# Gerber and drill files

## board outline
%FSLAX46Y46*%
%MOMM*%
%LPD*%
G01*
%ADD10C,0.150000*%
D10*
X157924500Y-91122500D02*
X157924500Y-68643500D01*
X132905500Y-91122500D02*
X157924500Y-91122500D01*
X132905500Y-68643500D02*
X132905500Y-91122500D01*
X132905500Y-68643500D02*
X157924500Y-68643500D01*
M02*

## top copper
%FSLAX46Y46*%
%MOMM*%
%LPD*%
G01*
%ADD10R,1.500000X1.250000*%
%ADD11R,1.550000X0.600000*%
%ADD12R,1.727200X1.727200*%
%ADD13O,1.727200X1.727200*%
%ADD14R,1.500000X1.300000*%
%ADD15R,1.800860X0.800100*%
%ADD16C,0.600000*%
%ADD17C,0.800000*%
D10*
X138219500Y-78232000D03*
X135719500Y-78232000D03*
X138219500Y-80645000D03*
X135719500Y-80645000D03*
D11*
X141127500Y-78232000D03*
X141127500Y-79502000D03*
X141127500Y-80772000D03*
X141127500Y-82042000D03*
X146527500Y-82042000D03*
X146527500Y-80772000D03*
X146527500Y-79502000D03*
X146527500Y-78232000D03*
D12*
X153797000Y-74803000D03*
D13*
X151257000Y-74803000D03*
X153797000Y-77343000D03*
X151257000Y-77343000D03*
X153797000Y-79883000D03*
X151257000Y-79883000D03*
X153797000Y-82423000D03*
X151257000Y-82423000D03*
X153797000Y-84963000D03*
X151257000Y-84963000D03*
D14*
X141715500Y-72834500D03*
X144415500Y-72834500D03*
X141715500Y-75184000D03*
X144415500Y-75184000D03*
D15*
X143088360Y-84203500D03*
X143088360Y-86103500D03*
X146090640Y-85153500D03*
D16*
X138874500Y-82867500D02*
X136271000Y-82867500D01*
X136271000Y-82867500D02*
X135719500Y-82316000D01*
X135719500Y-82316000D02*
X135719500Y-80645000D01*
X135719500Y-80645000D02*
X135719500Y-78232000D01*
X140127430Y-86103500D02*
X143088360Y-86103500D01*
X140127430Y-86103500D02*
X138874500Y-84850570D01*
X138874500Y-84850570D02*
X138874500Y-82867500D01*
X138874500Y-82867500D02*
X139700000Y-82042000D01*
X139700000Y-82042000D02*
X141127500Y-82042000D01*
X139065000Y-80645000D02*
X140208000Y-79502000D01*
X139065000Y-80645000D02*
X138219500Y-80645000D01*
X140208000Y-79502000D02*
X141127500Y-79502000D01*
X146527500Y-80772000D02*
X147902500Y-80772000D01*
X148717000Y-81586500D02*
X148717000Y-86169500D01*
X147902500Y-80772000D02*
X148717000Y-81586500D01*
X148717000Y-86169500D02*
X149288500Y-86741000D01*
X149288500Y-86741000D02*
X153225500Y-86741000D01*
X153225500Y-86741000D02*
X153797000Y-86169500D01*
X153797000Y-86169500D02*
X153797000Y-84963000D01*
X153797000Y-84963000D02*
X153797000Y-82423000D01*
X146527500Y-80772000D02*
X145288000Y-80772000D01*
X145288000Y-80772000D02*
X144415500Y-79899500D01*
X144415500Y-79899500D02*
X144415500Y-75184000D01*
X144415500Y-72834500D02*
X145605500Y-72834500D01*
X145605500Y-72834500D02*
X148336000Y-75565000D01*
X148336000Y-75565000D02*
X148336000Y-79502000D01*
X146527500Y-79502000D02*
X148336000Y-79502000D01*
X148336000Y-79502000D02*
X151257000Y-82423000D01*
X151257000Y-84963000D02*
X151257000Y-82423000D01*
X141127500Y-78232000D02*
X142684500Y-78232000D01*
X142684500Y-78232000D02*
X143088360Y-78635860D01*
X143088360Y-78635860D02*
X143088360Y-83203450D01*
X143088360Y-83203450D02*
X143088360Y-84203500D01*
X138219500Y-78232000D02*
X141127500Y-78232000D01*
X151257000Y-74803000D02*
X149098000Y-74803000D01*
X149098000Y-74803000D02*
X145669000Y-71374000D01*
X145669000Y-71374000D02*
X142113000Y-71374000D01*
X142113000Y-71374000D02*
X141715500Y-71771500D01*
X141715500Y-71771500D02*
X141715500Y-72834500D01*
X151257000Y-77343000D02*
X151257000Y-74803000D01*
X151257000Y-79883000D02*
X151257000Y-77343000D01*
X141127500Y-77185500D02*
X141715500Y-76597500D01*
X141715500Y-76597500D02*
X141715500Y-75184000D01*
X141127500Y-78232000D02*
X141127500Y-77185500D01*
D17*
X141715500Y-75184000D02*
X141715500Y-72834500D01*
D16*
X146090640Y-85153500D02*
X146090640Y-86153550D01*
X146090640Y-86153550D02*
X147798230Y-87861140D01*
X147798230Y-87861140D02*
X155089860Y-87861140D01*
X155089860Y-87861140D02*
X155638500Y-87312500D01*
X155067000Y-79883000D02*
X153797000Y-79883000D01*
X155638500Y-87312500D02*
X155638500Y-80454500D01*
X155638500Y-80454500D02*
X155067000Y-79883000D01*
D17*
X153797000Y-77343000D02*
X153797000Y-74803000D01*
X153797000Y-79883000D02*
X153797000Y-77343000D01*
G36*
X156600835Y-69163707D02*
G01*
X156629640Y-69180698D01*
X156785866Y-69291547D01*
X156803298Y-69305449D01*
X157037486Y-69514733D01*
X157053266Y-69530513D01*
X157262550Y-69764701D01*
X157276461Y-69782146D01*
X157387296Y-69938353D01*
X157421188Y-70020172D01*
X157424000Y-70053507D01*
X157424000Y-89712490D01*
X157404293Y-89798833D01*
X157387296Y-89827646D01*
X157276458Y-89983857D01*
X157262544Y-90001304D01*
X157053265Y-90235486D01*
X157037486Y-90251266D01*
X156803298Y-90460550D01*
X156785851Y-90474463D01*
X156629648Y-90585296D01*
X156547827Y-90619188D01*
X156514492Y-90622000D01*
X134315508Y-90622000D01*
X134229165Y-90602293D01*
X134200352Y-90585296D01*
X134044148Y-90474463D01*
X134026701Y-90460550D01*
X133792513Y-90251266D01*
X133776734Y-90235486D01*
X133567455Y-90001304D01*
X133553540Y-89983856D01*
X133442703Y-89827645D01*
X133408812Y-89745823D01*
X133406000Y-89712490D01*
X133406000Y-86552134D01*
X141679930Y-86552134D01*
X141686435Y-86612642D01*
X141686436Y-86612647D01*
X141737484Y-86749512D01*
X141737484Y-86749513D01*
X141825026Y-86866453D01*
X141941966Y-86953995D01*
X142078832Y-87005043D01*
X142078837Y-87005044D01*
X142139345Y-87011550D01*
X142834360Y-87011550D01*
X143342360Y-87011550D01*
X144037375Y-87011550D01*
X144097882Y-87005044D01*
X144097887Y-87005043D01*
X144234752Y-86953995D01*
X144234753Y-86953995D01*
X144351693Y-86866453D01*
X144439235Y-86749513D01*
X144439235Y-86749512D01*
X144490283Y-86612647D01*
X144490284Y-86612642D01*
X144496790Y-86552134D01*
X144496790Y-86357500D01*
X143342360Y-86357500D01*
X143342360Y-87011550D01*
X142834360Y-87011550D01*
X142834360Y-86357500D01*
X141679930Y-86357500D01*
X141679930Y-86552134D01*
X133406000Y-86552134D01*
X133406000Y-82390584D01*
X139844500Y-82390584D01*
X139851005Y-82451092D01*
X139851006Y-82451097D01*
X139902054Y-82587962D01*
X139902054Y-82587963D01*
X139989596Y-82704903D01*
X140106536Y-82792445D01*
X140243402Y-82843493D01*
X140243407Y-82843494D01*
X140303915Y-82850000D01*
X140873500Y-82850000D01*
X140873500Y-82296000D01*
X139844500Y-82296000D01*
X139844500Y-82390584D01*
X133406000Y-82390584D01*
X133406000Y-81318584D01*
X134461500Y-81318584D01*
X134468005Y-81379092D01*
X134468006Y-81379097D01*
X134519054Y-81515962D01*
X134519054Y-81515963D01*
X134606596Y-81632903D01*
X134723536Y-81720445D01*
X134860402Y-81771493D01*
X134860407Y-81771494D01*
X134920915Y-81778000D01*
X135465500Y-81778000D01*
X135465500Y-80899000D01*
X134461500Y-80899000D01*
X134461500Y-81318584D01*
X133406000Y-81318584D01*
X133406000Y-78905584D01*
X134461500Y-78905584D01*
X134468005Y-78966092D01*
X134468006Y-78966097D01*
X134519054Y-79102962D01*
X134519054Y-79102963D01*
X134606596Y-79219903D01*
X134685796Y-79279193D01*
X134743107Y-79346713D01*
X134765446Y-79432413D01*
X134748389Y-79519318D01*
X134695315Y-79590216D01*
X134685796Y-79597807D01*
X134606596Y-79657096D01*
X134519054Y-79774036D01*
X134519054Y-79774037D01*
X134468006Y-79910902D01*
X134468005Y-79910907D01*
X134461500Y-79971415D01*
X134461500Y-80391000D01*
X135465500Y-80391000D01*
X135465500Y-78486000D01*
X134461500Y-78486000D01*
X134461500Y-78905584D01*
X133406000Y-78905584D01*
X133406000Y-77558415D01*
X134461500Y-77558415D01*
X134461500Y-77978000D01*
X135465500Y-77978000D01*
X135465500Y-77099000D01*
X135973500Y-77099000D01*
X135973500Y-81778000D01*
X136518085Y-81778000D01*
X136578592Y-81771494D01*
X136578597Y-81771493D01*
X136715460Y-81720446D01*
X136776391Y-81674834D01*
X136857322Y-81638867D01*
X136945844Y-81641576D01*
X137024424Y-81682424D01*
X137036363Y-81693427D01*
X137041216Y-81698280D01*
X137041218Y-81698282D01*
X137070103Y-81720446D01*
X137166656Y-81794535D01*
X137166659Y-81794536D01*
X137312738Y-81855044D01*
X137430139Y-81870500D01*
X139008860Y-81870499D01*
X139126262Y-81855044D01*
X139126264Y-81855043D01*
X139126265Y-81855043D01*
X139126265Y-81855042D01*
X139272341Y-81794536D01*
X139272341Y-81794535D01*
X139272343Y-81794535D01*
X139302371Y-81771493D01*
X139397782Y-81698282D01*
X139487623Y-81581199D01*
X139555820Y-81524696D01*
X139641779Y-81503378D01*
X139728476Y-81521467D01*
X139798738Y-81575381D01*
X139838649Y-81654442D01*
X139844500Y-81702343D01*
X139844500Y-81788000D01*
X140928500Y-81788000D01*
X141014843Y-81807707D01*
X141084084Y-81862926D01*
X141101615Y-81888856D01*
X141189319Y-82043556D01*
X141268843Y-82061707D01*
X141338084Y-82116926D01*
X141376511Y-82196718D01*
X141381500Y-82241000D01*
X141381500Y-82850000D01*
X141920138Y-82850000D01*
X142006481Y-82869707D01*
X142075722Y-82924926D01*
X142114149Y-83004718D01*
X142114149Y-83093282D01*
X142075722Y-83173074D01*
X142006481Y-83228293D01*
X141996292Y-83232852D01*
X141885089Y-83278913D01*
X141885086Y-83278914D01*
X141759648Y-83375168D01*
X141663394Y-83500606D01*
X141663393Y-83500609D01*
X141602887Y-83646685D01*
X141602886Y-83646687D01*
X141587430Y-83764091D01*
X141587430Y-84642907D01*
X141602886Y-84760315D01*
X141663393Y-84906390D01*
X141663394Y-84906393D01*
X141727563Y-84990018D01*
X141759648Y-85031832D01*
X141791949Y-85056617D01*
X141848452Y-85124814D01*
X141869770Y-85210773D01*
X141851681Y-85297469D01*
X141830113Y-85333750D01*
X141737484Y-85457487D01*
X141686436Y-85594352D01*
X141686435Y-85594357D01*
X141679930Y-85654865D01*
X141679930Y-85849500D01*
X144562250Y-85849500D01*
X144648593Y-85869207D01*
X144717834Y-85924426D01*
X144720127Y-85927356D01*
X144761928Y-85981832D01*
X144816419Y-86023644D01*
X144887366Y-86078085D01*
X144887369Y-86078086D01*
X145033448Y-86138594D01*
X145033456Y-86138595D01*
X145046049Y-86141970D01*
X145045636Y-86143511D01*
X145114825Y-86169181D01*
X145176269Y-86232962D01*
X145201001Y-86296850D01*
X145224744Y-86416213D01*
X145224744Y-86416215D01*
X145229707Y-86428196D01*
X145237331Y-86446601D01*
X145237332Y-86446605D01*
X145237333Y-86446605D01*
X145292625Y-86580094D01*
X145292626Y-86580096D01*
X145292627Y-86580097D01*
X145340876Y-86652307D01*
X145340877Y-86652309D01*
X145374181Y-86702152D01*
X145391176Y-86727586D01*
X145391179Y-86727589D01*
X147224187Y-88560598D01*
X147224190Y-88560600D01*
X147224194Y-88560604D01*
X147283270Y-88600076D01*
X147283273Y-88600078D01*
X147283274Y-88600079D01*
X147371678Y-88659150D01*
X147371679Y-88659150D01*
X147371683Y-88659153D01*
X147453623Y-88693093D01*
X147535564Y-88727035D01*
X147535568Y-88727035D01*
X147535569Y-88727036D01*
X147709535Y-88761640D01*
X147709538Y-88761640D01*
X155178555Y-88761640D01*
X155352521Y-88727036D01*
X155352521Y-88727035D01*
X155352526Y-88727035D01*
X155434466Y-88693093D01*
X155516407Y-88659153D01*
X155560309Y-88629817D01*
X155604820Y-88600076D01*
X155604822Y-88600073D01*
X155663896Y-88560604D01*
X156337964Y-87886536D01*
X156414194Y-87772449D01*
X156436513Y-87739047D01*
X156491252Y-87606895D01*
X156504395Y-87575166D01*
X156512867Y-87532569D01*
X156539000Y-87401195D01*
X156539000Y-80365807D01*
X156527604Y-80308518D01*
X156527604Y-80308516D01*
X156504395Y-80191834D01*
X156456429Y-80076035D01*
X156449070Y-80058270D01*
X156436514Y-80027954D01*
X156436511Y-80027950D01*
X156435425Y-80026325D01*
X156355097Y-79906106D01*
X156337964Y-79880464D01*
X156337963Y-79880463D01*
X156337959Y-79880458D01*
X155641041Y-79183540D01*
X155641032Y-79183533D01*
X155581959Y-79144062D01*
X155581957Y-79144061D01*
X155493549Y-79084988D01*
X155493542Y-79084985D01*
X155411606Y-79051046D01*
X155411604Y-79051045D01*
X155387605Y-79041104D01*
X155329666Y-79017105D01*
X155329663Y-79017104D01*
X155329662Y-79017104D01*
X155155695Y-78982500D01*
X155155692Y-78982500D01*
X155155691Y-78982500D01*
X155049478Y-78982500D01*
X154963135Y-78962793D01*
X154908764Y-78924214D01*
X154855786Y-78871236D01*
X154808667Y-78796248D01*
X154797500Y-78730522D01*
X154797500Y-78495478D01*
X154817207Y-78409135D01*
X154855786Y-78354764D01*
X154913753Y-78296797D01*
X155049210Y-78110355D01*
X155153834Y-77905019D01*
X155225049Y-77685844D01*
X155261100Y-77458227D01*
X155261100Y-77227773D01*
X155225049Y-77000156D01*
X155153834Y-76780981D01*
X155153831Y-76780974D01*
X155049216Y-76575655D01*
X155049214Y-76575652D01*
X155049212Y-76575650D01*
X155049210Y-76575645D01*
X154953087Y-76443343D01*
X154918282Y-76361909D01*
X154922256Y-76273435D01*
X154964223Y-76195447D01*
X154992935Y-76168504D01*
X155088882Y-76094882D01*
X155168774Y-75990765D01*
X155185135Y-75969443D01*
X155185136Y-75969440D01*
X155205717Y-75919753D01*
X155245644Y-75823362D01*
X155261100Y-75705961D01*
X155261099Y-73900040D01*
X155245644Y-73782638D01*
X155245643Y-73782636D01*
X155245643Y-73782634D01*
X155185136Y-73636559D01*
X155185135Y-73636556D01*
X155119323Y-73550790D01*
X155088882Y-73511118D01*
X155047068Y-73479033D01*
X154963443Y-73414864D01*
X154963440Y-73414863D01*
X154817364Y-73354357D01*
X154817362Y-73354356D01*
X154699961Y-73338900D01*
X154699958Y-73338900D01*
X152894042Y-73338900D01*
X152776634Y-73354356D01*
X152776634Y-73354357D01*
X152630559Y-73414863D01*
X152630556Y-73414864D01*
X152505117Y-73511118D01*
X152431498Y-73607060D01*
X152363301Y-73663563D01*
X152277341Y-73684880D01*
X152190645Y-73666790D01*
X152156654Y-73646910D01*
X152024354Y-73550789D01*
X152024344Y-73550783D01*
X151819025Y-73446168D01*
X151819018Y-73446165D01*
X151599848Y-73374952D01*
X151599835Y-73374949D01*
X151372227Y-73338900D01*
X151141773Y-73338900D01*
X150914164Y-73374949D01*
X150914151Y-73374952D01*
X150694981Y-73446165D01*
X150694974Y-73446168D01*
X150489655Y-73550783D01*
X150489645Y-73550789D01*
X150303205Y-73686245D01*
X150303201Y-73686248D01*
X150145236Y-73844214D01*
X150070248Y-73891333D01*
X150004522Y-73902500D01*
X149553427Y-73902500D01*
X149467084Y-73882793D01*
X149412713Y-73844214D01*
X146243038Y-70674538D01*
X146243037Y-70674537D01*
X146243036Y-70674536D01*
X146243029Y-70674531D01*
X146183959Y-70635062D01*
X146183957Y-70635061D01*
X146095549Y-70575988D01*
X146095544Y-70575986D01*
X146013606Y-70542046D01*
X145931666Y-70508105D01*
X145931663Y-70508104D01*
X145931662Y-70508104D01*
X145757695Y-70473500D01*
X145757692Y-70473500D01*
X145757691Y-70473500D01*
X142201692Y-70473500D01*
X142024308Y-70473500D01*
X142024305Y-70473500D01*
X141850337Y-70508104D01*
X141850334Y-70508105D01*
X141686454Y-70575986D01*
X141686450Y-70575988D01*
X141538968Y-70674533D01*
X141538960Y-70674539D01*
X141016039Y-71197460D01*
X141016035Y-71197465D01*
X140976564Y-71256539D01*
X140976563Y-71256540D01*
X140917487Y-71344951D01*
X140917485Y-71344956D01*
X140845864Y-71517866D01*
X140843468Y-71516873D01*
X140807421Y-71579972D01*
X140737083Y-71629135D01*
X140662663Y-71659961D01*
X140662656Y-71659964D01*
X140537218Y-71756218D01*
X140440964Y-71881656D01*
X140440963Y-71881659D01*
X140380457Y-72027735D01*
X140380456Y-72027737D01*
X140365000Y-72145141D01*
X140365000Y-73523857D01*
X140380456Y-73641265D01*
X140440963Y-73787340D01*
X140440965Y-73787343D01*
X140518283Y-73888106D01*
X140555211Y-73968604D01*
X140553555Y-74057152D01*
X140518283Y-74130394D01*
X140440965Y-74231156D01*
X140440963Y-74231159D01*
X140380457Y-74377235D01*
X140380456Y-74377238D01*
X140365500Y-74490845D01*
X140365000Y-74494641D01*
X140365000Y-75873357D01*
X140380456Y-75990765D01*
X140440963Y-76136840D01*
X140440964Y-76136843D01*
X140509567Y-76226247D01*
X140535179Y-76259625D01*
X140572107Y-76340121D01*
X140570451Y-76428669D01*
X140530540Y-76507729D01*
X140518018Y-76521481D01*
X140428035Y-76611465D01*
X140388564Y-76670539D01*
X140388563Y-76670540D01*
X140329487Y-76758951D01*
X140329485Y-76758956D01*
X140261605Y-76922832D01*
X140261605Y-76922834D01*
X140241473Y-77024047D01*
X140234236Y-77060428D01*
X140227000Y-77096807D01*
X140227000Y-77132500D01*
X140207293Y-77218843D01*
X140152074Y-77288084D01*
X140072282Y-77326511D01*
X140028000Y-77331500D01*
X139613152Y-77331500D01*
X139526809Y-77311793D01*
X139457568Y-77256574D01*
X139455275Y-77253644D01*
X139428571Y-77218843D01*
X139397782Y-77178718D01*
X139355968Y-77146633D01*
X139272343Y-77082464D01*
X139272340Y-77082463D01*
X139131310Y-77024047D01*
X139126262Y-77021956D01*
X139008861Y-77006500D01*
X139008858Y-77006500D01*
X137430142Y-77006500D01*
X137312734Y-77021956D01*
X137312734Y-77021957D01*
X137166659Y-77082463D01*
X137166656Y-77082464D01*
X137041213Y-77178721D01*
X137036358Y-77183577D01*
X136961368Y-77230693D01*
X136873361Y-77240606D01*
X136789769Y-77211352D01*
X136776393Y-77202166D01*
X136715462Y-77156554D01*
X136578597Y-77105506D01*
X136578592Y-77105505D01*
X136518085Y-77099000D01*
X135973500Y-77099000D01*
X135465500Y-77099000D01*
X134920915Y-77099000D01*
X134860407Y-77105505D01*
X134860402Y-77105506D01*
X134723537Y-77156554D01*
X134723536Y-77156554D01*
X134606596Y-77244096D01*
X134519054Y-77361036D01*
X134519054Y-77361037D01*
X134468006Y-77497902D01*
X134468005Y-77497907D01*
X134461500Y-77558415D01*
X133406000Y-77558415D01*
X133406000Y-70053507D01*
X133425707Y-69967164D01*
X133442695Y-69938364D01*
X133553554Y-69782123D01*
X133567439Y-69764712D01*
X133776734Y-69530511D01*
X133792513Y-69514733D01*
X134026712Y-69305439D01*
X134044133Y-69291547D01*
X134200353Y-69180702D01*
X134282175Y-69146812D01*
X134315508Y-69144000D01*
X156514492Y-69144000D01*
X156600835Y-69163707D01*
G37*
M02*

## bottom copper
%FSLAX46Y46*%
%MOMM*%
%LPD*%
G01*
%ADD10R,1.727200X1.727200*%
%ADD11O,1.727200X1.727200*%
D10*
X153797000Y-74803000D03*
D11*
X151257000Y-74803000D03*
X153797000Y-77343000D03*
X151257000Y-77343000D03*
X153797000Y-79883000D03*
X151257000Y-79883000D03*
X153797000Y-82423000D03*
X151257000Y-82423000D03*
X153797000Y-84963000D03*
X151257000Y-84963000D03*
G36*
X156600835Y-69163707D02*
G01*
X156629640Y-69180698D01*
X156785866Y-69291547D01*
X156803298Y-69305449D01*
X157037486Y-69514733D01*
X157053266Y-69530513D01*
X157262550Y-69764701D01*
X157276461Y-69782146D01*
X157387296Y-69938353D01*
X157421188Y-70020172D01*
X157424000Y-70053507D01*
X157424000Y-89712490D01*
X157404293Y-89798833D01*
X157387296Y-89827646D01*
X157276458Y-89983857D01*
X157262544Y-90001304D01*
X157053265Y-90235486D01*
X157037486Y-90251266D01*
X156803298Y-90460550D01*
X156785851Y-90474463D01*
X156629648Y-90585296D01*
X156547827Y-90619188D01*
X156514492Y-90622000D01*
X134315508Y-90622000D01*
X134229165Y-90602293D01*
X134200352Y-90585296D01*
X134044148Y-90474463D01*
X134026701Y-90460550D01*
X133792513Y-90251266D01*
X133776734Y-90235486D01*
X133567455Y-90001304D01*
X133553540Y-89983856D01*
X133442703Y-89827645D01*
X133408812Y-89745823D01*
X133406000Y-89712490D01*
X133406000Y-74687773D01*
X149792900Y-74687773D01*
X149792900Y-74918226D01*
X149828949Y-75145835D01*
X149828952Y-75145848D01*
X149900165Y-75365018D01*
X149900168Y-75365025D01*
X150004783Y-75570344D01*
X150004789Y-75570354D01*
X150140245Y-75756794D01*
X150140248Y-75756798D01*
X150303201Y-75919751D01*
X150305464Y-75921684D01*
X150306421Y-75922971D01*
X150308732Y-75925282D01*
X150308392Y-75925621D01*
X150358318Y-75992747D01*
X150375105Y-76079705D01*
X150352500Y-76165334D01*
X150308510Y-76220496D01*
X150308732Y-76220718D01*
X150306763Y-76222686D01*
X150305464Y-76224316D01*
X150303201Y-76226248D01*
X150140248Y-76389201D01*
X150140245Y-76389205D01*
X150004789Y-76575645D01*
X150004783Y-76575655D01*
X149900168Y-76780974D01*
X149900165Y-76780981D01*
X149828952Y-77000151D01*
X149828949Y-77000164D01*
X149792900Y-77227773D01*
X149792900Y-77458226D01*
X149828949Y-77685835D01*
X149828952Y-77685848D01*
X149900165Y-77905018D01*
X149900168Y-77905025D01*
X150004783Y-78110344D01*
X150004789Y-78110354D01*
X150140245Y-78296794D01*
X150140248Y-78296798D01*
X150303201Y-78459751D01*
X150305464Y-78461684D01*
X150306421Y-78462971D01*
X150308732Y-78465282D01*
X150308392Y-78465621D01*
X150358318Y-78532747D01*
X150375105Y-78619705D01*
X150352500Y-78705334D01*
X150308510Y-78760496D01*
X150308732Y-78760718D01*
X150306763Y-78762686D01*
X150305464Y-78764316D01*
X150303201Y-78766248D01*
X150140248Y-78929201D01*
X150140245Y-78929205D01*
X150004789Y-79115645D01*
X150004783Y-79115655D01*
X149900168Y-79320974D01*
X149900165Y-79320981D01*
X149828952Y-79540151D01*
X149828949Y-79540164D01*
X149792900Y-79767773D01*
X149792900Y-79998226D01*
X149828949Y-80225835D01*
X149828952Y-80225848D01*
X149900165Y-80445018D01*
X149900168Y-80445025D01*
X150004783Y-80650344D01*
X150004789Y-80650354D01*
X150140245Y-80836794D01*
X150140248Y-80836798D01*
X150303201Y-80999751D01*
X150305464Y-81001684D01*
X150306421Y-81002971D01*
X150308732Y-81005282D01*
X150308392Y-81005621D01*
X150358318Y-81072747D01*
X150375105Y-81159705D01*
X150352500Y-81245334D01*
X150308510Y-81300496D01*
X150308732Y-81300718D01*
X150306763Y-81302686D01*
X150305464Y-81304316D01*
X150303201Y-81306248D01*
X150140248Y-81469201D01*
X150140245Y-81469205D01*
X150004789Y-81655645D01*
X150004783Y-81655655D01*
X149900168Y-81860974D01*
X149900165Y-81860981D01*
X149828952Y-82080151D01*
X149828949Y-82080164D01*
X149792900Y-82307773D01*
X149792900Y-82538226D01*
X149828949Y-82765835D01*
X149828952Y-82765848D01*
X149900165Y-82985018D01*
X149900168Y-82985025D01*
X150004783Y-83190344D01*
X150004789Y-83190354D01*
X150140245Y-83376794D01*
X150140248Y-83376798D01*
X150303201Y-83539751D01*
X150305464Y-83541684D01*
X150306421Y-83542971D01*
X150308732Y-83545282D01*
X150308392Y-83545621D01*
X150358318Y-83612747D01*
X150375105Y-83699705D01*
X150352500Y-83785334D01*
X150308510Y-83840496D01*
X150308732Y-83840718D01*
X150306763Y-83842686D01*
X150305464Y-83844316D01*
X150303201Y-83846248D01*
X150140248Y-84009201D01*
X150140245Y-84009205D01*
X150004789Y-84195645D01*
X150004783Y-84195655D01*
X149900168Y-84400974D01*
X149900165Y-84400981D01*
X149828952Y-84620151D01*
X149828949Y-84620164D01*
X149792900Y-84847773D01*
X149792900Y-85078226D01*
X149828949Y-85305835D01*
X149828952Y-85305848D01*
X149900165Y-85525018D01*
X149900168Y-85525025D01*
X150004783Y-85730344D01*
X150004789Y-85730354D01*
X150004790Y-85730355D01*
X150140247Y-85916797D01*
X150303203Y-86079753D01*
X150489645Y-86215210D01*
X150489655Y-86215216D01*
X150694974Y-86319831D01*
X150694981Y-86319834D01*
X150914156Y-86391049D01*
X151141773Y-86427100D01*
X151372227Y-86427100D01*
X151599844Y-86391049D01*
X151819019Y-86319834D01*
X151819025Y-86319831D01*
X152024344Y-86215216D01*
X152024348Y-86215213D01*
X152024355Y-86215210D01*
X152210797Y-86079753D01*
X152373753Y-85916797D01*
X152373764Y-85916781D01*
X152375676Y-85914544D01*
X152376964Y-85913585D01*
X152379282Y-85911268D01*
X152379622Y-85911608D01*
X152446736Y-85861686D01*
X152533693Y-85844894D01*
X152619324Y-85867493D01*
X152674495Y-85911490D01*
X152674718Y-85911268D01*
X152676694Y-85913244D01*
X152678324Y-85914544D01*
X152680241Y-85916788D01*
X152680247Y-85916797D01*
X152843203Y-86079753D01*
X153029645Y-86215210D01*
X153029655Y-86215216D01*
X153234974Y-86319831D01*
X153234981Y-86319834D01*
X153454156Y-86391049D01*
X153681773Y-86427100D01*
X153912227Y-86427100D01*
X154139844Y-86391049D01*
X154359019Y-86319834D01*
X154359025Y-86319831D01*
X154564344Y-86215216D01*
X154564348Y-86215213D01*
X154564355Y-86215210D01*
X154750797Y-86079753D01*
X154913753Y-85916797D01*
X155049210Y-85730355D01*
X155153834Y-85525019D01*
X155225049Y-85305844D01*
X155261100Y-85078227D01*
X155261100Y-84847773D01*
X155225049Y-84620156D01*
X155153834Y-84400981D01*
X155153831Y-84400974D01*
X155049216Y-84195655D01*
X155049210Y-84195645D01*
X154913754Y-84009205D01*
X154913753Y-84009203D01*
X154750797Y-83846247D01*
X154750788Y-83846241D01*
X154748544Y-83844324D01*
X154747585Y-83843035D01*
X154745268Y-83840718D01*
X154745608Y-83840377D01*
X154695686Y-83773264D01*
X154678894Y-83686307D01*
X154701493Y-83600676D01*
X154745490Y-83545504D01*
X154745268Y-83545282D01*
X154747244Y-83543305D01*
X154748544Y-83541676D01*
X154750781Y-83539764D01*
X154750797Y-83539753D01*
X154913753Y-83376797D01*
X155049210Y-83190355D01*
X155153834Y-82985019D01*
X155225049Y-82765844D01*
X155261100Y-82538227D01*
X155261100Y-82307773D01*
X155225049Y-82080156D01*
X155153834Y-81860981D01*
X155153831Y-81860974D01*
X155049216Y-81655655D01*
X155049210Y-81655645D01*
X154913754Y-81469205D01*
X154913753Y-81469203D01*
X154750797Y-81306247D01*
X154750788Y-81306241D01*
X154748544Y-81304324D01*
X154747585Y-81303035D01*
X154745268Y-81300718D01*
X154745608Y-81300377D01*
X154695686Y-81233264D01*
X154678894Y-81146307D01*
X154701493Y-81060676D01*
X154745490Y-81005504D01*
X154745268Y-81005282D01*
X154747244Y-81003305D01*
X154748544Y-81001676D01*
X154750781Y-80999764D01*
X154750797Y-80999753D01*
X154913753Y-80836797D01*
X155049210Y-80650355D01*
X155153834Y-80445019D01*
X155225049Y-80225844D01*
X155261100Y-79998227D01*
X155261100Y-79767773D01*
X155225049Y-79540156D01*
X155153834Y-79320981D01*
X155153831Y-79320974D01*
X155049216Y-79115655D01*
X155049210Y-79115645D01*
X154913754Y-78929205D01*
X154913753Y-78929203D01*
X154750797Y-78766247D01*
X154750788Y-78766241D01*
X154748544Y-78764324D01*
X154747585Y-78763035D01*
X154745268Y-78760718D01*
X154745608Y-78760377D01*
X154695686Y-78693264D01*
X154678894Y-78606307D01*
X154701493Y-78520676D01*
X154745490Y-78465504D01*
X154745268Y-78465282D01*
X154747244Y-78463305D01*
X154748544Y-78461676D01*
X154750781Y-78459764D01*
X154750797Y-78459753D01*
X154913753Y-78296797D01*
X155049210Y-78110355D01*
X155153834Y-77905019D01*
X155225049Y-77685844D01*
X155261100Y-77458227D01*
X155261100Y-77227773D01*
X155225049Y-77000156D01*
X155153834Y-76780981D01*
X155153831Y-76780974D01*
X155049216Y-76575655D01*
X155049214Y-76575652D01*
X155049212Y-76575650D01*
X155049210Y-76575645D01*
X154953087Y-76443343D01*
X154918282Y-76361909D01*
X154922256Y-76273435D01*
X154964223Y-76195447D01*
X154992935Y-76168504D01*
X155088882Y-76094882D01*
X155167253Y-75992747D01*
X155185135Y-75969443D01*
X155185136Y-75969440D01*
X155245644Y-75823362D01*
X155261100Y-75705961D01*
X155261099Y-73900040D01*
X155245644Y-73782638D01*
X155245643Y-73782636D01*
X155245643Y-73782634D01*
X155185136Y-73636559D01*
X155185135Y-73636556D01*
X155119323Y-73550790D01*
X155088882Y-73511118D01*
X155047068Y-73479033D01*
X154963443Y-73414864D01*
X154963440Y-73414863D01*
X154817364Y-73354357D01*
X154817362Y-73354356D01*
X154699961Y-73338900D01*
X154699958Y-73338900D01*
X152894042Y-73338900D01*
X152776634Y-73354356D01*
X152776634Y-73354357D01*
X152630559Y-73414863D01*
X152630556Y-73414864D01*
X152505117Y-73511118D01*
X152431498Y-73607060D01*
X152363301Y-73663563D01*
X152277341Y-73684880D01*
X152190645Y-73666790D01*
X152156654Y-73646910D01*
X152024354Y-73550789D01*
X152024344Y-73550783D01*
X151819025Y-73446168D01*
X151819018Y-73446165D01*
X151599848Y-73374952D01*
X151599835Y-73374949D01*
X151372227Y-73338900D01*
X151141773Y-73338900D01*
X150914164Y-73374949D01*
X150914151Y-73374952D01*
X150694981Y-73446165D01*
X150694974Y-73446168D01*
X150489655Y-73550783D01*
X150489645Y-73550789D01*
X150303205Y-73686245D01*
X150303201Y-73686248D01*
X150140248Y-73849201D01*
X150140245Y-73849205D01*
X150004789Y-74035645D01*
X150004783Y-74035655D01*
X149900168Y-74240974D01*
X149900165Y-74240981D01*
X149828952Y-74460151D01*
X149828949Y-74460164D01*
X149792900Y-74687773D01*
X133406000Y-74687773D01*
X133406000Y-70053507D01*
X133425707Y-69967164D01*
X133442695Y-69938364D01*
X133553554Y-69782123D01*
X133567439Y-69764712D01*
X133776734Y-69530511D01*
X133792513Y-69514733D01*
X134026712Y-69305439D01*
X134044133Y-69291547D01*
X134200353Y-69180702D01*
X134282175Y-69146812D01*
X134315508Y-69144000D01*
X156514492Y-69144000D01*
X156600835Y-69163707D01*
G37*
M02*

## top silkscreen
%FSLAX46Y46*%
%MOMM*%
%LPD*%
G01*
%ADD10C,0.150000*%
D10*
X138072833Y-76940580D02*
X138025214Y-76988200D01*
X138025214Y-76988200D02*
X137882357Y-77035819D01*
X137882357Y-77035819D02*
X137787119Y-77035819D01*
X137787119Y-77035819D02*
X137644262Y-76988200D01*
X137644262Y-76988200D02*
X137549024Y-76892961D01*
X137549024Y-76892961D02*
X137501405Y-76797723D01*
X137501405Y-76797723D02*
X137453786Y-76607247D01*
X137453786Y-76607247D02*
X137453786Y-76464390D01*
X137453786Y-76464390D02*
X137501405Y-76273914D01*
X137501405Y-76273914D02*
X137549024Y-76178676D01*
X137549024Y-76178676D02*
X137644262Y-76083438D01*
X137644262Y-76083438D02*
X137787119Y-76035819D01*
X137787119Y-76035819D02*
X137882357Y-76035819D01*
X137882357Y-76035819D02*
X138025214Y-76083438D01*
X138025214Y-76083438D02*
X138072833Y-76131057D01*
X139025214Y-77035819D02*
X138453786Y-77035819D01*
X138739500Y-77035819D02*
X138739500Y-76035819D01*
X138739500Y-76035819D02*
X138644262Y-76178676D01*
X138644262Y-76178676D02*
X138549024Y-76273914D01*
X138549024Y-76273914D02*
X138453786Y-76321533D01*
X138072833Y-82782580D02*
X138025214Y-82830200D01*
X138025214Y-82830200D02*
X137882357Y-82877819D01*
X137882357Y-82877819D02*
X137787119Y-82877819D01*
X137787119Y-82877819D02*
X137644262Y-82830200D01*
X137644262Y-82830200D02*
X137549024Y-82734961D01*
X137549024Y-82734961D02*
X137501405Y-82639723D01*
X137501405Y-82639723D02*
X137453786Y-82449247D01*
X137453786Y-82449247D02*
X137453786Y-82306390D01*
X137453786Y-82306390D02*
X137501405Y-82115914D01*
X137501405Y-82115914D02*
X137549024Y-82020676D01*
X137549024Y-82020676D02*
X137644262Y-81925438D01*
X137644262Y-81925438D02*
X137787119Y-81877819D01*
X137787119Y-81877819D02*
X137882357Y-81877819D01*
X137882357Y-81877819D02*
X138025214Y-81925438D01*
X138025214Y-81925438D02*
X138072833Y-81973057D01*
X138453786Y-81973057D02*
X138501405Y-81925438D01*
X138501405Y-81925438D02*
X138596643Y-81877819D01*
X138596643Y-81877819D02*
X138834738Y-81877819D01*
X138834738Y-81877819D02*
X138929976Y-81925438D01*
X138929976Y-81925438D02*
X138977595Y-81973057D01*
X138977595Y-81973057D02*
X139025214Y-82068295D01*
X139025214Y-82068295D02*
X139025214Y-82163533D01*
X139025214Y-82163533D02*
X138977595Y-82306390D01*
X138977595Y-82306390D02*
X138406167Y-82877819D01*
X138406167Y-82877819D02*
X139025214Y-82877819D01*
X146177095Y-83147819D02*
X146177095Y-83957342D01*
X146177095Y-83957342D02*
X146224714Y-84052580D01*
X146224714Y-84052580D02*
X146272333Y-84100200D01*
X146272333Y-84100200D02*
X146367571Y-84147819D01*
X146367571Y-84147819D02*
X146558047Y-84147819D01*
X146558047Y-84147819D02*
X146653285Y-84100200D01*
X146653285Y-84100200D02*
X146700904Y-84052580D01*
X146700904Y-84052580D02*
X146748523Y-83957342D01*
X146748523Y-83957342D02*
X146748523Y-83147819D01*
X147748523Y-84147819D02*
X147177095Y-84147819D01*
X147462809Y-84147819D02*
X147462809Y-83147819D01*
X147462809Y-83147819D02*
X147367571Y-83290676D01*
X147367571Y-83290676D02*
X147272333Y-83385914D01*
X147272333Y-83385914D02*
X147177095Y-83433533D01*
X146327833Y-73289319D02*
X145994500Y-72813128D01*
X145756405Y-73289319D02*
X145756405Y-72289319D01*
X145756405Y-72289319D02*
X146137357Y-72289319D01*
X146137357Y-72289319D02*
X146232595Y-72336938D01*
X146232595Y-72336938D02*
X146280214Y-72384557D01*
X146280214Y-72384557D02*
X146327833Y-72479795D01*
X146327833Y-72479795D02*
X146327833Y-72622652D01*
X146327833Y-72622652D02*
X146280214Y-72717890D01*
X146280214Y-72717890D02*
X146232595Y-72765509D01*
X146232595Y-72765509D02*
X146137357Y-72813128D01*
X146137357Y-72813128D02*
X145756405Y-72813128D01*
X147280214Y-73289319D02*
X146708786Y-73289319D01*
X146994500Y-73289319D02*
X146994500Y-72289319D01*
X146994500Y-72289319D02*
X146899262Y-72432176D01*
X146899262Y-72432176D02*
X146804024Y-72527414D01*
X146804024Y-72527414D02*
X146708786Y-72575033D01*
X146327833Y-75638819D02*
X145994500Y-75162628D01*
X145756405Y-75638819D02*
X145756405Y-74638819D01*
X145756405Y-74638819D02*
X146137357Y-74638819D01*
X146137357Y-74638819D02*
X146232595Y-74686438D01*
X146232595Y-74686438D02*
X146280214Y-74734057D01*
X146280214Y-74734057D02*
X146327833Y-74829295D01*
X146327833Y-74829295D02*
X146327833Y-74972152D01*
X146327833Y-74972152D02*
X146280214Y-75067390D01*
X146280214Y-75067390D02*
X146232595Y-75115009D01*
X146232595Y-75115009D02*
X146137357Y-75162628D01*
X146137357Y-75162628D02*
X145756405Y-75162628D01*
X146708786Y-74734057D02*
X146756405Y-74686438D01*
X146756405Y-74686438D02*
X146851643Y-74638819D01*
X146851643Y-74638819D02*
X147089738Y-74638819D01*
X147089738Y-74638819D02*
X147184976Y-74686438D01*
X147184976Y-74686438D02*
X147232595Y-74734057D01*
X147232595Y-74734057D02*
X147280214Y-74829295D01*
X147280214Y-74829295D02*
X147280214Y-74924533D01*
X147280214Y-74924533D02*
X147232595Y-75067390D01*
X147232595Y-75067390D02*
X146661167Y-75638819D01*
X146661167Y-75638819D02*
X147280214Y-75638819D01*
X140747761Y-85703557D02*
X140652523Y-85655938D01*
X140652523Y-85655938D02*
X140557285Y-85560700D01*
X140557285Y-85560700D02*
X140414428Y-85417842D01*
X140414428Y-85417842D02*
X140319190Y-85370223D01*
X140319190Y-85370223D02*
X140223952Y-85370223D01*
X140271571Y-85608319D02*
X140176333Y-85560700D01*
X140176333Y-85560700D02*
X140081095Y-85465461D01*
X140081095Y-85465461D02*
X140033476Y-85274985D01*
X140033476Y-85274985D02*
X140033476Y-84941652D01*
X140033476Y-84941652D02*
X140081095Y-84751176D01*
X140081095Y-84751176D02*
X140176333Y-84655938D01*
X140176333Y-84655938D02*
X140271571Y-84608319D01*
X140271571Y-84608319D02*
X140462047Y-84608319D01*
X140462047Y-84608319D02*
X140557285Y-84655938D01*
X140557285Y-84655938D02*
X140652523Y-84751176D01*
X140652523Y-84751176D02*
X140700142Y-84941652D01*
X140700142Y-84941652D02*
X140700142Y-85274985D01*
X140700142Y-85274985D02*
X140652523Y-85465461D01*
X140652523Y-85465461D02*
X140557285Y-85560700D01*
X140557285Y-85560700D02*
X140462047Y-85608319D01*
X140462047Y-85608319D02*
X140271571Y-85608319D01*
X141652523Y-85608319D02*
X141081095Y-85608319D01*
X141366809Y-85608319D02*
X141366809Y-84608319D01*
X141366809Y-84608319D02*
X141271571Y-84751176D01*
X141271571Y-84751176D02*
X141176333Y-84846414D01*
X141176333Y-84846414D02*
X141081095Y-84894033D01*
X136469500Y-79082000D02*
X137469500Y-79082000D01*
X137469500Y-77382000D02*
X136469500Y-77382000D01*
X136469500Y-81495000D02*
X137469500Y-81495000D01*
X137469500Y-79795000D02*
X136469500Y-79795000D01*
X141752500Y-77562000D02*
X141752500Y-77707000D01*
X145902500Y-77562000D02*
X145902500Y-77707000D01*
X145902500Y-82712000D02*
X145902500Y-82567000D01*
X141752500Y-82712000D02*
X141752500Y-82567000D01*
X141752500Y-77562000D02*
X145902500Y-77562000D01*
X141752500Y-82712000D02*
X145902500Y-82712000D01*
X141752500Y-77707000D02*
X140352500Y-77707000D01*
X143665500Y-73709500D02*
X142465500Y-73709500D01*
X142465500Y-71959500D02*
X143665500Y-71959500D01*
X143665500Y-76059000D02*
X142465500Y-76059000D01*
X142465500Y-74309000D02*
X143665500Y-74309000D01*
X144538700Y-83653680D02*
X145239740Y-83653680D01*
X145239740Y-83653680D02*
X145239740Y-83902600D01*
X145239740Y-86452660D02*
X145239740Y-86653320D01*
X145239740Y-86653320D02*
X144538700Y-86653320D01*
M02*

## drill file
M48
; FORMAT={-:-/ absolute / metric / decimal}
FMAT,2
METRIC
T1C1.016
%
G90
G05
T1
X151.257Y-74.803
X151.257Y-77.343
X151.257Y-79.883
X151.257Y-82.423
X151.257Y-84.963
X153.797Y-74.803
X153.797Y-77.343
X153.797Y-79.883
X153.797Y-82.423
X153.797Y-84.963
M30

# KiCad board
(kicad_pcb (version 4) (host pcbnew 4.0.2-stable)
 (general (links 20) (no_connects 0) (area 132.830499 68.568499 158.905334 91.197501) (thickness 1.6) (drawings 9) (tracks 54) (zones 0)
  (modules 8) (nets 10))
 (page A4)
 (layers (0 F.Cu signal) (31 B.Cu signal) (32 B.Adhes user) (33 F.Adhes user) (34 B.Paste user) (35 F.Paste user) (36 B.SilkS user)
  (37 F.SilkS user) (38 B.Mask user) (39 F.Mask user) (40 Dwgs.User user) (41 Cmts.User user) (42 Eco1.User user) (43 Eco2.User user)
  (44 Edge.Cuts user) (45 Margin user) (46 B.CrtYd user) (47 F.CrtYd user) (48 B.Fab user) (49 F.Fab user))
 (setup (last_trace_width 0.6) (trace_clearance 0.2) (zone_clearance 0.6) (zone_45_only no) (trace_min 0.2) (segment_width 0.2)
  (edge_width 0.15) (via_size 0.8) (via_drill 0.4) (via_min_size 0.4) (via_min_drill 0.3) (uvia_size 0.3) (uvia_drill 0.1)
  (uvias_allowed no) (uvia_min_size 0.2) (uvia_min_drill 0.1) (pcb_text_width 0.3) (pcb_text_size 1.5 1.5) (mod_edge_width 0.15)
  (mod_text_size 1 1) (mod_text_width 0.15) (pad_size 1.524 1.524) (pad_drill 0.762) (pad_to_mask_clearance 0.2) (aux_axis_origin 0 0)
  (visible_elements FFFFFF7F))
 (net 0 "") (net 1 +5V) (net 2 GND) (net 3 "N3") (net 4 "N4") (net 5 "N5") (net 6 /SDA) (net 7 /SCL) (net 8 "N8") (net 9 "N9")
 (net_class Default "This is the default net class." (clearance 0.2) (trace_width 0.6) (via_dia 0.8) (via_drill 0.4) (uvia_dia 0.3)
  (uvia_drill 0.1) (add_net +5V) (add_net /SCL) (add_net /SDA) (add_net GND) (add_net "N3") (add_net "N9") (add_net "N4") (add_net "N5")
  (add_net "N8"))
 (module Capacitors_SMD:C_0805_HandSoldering (layer F.Cu) (at 136.9695 78.232 180)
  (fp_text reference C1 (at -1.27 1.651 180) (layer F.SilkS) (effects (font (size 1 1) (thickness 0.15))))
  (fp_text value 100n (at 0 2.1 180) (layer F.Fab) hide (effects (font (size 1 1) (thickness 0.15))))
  (fp_line (start 0.5 -0.85) (end -0.5 -0.85) (layer F.SilkS) (width 0.15))
  (fp_line (start -0.5 0.85) (end 0.5 0.85) (layer F.SilkS) (width 0.15))
  (pad 1 smd rect (at -1.25 0 180) (size 1.5 1.25) (layers F.Cu F.Paste F.Mask) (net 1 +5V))
  (pad 2 smd rect (at 1.25 0 180) (size 1.5 1.25) (layers F.Cu F.Paste F.Mask) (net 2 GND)))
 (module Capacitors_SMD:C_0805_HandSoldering (layer F.Cu) (at 136.9695 80.645 180)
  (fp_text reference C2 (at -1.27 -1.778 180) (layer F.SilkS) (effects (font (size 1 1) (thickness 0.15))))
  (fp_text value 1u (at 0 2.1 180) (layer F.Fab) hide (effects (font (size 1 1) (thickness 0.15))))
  (fp_line (start 0.5 -0.85) (end -0.5 -0.85) (layer F.SilkS) (width 0.15))
  (fp_line (start -0.5 0.85) (end 0.5 0.85) (layer F.SilkS) (width 0.15))
  (pad 1 smd rect (at -1.25 0 180) (size 1.5 1.25) (layers F.Cu F.Paste F.Mask) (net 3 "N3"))
  (pad 2 smd rect (at 1.25 0 180) (size 1.5 1.25) (layers F.Cu F.Paste F.Mask) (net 2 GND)))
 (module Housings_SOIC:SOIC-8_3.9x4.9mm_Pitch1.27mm (layer F.Cu) (at 143.8275 80.137)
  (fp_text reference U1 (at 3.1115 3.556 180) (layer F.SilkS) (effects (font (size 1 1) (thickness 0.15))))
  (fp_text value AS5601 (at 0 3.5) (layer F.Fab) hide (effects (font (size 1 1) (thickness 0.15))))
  (fp_line (start -2.075 -2.575) (end -2.075 -2.43) (layer F.SilkS) (width 0.15))
  (fp_line (start 2.075 -2.575) (end 2.075 -2.43) (layer F.SilkS) (width 0.15))
  (fp_line (start 2.075 2.575) (end 2.075 2.43) (layer F.SilkS) (width 0.15))
  (fp_line (start -2.075 2.575) (end -2.075 2.43) (layer F.SilkS) (width 0.15))
  (fp_line (start -2.075 -2.575) (end 2.075 -2.575) (layer F.SilkS) (width 0.15))
  (fp_line (start -2.075 2.575) (end 2.075 2.575) (layer F.SilkS) (width 0.15))
  (fp_line (start -2.075 -2.43) (end -3.475 -2.43) (layer F.SilkS) (width 0.15))
  (pad 1 smd rect (at -2.7 -1.905) (size 1.55 0.6) (layers F.Cu F.Paste F.Mask) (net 1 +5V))
  (pad 2 smd rect (at -2.7 -0.635) (size 1.55 0.6) (layers F.Cu F.Paste F.Mask) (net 3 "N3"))
  (pad 3 smd rect (at -2.7 0.635) (size 1.55 0.6) (layers F.Cu F.Paste F.Mask) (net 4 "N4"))
  (pad 4 smd rect (at -2.7 1.905) (size 1.55 0.6) (layers F.Cu F.Paste F.Mask) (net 2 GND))
  (pad 5 smd rect (at 2.7 1.905) (size 1.55 0.6) (layers F.Cu F.Paste F.Mask) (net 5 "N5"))
  (pad 6 smd rect (at 2.7 0.635) (size 1.55 0.6) (layers F.Cu F.Paste F.Mask) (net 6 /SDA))
  (pad 7 smd rect (at 2.7 -0.635) (size 1.55 0.6) (layers F.Cu F.Paste F.Mask) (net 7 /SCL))
  (pad 8 smd rect (at 2.7 -1.905) (size 1.55 0.6) (layers F.Cu F.Paste F.Mask) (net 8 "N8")))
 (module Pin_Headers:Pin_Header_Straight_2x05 (layer B.Cu) (at 153.797 74.803 180)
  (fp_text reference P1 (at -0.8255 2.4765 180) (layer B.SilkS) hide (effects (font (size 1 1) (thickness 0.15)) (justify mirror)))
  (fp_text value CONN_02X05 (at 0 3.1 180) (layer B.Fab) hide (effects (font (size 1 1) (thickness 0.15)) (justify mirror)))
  (pad 1 thru_hole rect (at 0 0 180) (size 1.7272 1.7272) (drill 1.016) (layers *.Cu *.Mask B.SilkS) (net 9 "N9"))
  (pad 2 thru_hole oval (at 2.54 0 180) (size 1.7272 1.7272) (drill 1.016) (layers *.Cu *.Mask B.SilkS) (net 1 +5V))
  (pad 3 thru_hole oval (at 0 -2.54 180) (size 1.7272 1.7272) (drill 1.016) (layers *.Cu *.Mask B.SilkS) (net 9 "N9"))
  (pad 4 thru_hole oval (at 2.54 -2.54 180) (size 1.7272 1.7272) (drill 1.016) (layers *.Cu *.Mask B.SilkS) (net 1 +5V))
  (pad 5 thru_hole oval (at 0 -5.08 180) (size 1.7272 1.7272) (drill 1.016) (layers *.Cu *.Mask B.SilkS) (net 9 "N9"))
  (pad 6 thru_hole oval (at 2.54 -5.08 180) (size 1.7272 1.7272) (drill 1.016) (layers *.Cu *.Mask B.SilkS) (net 1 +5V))
  (pad 7 thru_hole oval (at 0 -7.62 180) (size 1.7272 1.7272) (drill 1.016) (layers *.Cu *.Mask B.SilkS) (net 6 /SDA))
  (pad 8 thru_hole oval (at 2.54 -7.62 180) (size 1.7272 1.7272) (drill 1.016) (layers *.Cu *.Mask B.SilkS) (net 7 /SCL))
  (pad 9 thru_hole oval (at 0 -10.16 180) (size 1.7272 1.7272) (drill 1.016) (layers *.Cu *.Mask B.SilkS) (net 6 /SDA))
  (pad 10 thru_hole oval (at 2.54 -10.16 180) (size 1.7272 1.7272) (drill 1.016) (layers *.Cu *.Mask B.SilkS) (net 7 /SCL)))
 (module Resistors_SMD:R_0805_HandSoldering (layer F.Cu) (at 143.0655 72.8345)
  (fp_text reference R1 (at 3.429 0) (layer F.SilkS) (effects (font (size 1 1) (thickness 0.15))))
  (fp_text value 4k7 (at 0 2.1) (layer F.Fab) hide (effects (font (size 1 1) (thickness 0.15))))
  (fp_line (start 0.6 0.875) (end -0.6 0.875) (layer F.SilkS) (width 0.15))
  (fp_line (start -0.6 -0.875) (end 0.6 -0.875) (layer F.SilkS) (width 0.15))
  (pad 1 smd rect (at -1.35 0) (size 1.5 1.3) (layers F.Cu F.Paste F.Mask) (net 1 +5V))
  (pad 2 smd rect (at 1.35 0) (size 1.5 1.3) (layers F.Cu F.Paste F.Mask) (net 7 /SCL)))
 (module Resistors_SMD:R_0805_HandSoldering (layer F.Cu) (at 143.0655 75.184)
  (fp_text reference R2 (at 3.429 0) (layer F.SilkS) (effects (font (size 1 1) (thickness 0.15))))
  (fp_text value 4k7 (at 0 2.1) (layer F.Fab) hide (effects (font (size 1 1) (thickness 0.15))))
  (fp_line (start 0.6 0.875) (end -0.6 0.875) (layer F.SilkS) (width 0.15))
  (fp_line (start -0.6 -0.875) (end 0.6 -0.875) (layer F.SilkS) (width 0.15))
  (pad 1 smd rect (at -1.35 0) (size 1.5 1.3) (layers F.Cu F.Paste F.Mask) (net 1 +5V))
  (pad 2 smd rect (at 1.35 0) (size 1.5 1.3) (layers F.Cu F.Paste F.Mask) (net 6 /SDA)))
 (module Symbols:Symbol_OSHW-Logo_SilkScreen (layer B.Cu) (at 137.8839 79.3115 180)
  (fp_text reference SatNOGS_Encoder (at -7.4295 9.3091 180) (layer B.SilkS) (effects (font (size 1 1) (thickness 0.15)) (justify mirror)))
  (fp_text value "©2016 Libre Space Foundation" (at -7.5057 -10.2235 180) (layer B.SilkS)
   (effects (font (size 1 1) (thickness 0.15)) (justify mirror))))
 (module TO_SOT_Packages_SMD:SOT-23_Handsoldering (layer F.Cu) (at 144.5895 85.1535 270)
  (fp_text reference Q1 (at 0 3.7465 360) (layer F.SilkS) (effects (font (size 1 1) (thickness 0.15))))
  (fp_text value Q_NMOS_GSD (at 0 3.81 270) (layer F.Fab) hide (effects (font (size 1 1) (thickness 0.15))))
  (fp_line (start -1.49982 0.0508) (end -1.49982 -0.65024) (layer F.SilkS) (width 0.15))
  (fp_line (start -1.49982 -0.65024) (end -1.2509 -0.65024) (layer F.SilkS) (width 0.15))
  (fp_line (start 1.29916 -0.65024) (end 1.49982 -0.65024) (layer F.SilkS) (width 0.15))
  (fp_line (start 1.49982 -0.65024) (end 1.49982 0.0508) (layer F.SilkS) (width 0.15))
  (pad 1 smd rect (at -0.95 1.50114 270) (size 0.8001 1.80086) (layers F.Cu F.Paste F.Mask) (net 1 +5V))
  (pad 2 smd rect (at 0.95 1.50114 270) (size 0.8001 1.80086) (layers F.Cu F.Paste F.Mask) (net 2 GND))
  (pad 3 smd rect (at 0 -1.50114 270) (size 0.8001 1.80086) (layers F.Cu F.Paste F.Mask) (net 9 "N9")))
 (gr_line (start 157.9245 91.1225) (end 157.9245 68.6435) (layer Edge.Cuts) (width 0.15))
 (gr_line (start 132.9055 91.1225) (end 157.9245 91.1225) (layer Edge.Cuts) (width 0.15))
 (gr_line (start 132.9055 68.6435) (end 132.9055 91.1225) (layer Edge.Cuts) (width 0.15))
 (gr_line (start 132.9055 68.6435) (end 157.9245 68.6435) (layer Edge.Cuts) (width 0.15))
 (segment (start 138.8745 82.8675) (end 136.271 82.8675) (width 0.6) (layer F.Cu) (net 2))
 (segment (start 136.271 82.8675) (end 135.7195 82.316) (width 0.6) (layer F.Cu) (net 2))
 (segment (start 135.7195 82.316) (end 135.7195 80.645) (width 0.6) (layer F.Cu) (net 2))
 (segment (start 135.7195 80.645) (end 135.7195 78.232) (width 0.6) (layer F.Cu) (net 2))
 (segment (start 140.12743 86.1035) (end 143.08836 86.1035) (width 0.6) (layer F.Cu) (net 2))
 (segment (start 140.12743 86.1035) (end 138.8745 84.85057) (width 0.6) (layer F.Cu) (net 2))
 (segment (start 138.8745 84.85057) (end 138.8745 82.8675) (width 0.6) (layer F.Cu) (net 2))
 (segment (start 138.8745 82.8675) (end 139.7 82.042) (width 0.6) (layer F.Cu) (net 2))
 (segment (start 139.7 82.042) (end 141.1275 82.042) (width 0.6) (layer F.Cu) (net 2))
 (segment (start 139.065 80.645) (end 140.208 79.502) (width 0.6) (layer F.Cu) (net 3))
 (segment (start 139.065 80.645) (end 138.2195 80.645) (width 0.6) (layer F.Cu) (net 3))
 (segment (start 140.208 79.502) (end 141.1275 79.502) (width 0.6) (layer F.Cu) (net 3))
 (segment (start 146.5275 80.772) (end 147.9025 80.772) (width 0.6) (layer F.Cu) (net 6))
 (segment (start 148.717 81.5865) (end 148.717 86.1695) (width 0.6) (layer F.Cu) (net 6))
 (segment (start 147.9025 80.772) (end 148.717 81.5865) (width 0.6) (layer F.Cu) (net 6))
 (segment (start 148.717 86.1695) (end 149.2885 86.741) (width 0.6) (layer F.Cu) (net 6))
 (segment (start 149.2885 86.741) (end 153.2255 86.741) (width 0.6) (layer F.Cu) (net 6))
 (segment (start 153.2255 86.741) (end 153.797 86.1695) (width 0.6) (layer F.Cu) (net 6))
 (segment (start 153.797 86.1695) (end 153.797 84.963) (width 0.6) (layer F.Cu) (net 6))
 (segment (start 153.797 84.963) (end 153.797 82.423) (width 0.6) (layer F.Cu) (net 6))
 (segment (start 146.5275 80.772) (end 145.288 80.772) (width 0.6) (layer F.Cu) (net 6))
 (segment (start 145.288 80.772) (end 144.4155 79.8995) (width 0.6) (layer F.Cu) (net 6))
 (segment (start 144.4155 79.8995) (end 144.4155 75.184) (width 0.6) (layer F.Cu) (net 6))
 (segment (start 144.4155 72.8345) (end 145.6055 72.8345) (width 0.6) (layer F.Cu) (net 7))
 (segment (start 145.6055 72.8345) (end 148.336 75.565) (width 0.6) (layer F.Cu) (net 7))
 (segment (start 148.336 75.565) (end 148.336 79.502) (width 0.6) (layer F.Cu) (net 7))
 (segment (start 146.5275 79.502) (end 148.336 79.502) (width 0.6) (layer F.Cu) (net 7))
 (segment (start 148.336 79.502) (end 151.257 82.423) (width 0.6) (layer F.Cu) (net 7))
 (segment (start 151.257 84.963) (end 151.257 82.423) (width 0.6) (layer F.Cu) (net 7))
 (segment (start 141.1275 78.232) (end 142.6845 78.232) (width 0.6) (layer F.Cu) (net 1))
 (segment (start 142.6845 78.232) (end 143.08836 78.63586) (width 0.6) (layer F.Cu) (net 1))
 (segment (start 143.08836 78.63586) (end 143.08836 83.20345) (width 0.6) (layer F.Cu) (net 1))
 (segment (start 143.08836 83.20345) (end 143.08836 84.2035) (width 0.6) (layer F.Cu) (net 1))
 (segment (start 138.2195 78.232) (end 141.1275 78.232) (width 0.6) (layer F.Cu) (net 1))
 (segment (start 151.257 74.803) (end 149.098 74.803) (width 0.6) (layer F.Cu) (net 1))
 (segment (start 149.098 74.803) (end 145.669 71.374) (width 0.6) (layer F.Cu) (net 1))
 (segment (start 145.669 71.374) (end 142.113 71.374) (width 0.6) (layer F.Cu) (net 1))
 (segment (start 142.113 71.374) (end 141.7155 71.7715) (width 0.6) (layer F.Cu) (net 1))
 (segment (start 141.7155 71.7715) (end 141.7155 72.8345) (width 0.6) (layer F.Cu) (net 1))
 (segment (start 151.257 77.343) (end 151.257 74.803) (width 0.6) (layer F.Cu) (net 1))
 (segment (start 151.257 79.883) (end 151.257 77.343) (width 0.6) (layer F.Cu) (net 1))
 (segment (start 141.1275 77.1855) (end 141.7155 76.5975) (width 0.6) (layer F.Cu) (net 1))
 (segment (start 141.7155 76.5975) (end 141.7155 75.184) (width 0.6) (layer F.Cu) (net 1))
 (segment (start 141.1275 78.232) (end 141.1275 77.1855) (width 0.6) (layer F.Cu) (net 1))
 (segment (start 141.7155 75.184) (end 141.7155 72.8345) (width 0.8) (layer F.Cu) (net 1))
 (segment (start 146.09064 85.1535) (end 146.09064 86.15355) (width 0.6) (layer F.Cu) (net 9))
 (segment (start 146.09064 86.15355) (end 147.79823 87.86114) (width 0.6) (layer F.Cu) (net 9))
 (segment (start 147.79823 87.86114) (end 155.08986 87.86114) (width 0.6) (layer F.Cu) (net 9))
 (segment (start 155.08986 87.86114) (end 155.6385 87.3125) (width 0.6) (layer F.Cu) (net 9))
 (segment (start 155.067 79.883) (end 153.797 79.883) (width 0.6) (layer F.Cu) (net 9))
 (segment (start 155.6385 87.3125) (end 155.6385 80.4545) (width 0.6) (layer F.Cu) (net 9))
 (segment (start 155.6385 80.4545) (end 155.067 79.883) (width 0.6) (layer F.Cu) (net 9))
 (segment (start 153.797 77.343) (end 153.797 74.803) (width 0.8) (layer F.Cu) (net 9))
 (segment (start 153.797 79.883) (end 153.797 77.343) (width 0.8) (layer F.Cu) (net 9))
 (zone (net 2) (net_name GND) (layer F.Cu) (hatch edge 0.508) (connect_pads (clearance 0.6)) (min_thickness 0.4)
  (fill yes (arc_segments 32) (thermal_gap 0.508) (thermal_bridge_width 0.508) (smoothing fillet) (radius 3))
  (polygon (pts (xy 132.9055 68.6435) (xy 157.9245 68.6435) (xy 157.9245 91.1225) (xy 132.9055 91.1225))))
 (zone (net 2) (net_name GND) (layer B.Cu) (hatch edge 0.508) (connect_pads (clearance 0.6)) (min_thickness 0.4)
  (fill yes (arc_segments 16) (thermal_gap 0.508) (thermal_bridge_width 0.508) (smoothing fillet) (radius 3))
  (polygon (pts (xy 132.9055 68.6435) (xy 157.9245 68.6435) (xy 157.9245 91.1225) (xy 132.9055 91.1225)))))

